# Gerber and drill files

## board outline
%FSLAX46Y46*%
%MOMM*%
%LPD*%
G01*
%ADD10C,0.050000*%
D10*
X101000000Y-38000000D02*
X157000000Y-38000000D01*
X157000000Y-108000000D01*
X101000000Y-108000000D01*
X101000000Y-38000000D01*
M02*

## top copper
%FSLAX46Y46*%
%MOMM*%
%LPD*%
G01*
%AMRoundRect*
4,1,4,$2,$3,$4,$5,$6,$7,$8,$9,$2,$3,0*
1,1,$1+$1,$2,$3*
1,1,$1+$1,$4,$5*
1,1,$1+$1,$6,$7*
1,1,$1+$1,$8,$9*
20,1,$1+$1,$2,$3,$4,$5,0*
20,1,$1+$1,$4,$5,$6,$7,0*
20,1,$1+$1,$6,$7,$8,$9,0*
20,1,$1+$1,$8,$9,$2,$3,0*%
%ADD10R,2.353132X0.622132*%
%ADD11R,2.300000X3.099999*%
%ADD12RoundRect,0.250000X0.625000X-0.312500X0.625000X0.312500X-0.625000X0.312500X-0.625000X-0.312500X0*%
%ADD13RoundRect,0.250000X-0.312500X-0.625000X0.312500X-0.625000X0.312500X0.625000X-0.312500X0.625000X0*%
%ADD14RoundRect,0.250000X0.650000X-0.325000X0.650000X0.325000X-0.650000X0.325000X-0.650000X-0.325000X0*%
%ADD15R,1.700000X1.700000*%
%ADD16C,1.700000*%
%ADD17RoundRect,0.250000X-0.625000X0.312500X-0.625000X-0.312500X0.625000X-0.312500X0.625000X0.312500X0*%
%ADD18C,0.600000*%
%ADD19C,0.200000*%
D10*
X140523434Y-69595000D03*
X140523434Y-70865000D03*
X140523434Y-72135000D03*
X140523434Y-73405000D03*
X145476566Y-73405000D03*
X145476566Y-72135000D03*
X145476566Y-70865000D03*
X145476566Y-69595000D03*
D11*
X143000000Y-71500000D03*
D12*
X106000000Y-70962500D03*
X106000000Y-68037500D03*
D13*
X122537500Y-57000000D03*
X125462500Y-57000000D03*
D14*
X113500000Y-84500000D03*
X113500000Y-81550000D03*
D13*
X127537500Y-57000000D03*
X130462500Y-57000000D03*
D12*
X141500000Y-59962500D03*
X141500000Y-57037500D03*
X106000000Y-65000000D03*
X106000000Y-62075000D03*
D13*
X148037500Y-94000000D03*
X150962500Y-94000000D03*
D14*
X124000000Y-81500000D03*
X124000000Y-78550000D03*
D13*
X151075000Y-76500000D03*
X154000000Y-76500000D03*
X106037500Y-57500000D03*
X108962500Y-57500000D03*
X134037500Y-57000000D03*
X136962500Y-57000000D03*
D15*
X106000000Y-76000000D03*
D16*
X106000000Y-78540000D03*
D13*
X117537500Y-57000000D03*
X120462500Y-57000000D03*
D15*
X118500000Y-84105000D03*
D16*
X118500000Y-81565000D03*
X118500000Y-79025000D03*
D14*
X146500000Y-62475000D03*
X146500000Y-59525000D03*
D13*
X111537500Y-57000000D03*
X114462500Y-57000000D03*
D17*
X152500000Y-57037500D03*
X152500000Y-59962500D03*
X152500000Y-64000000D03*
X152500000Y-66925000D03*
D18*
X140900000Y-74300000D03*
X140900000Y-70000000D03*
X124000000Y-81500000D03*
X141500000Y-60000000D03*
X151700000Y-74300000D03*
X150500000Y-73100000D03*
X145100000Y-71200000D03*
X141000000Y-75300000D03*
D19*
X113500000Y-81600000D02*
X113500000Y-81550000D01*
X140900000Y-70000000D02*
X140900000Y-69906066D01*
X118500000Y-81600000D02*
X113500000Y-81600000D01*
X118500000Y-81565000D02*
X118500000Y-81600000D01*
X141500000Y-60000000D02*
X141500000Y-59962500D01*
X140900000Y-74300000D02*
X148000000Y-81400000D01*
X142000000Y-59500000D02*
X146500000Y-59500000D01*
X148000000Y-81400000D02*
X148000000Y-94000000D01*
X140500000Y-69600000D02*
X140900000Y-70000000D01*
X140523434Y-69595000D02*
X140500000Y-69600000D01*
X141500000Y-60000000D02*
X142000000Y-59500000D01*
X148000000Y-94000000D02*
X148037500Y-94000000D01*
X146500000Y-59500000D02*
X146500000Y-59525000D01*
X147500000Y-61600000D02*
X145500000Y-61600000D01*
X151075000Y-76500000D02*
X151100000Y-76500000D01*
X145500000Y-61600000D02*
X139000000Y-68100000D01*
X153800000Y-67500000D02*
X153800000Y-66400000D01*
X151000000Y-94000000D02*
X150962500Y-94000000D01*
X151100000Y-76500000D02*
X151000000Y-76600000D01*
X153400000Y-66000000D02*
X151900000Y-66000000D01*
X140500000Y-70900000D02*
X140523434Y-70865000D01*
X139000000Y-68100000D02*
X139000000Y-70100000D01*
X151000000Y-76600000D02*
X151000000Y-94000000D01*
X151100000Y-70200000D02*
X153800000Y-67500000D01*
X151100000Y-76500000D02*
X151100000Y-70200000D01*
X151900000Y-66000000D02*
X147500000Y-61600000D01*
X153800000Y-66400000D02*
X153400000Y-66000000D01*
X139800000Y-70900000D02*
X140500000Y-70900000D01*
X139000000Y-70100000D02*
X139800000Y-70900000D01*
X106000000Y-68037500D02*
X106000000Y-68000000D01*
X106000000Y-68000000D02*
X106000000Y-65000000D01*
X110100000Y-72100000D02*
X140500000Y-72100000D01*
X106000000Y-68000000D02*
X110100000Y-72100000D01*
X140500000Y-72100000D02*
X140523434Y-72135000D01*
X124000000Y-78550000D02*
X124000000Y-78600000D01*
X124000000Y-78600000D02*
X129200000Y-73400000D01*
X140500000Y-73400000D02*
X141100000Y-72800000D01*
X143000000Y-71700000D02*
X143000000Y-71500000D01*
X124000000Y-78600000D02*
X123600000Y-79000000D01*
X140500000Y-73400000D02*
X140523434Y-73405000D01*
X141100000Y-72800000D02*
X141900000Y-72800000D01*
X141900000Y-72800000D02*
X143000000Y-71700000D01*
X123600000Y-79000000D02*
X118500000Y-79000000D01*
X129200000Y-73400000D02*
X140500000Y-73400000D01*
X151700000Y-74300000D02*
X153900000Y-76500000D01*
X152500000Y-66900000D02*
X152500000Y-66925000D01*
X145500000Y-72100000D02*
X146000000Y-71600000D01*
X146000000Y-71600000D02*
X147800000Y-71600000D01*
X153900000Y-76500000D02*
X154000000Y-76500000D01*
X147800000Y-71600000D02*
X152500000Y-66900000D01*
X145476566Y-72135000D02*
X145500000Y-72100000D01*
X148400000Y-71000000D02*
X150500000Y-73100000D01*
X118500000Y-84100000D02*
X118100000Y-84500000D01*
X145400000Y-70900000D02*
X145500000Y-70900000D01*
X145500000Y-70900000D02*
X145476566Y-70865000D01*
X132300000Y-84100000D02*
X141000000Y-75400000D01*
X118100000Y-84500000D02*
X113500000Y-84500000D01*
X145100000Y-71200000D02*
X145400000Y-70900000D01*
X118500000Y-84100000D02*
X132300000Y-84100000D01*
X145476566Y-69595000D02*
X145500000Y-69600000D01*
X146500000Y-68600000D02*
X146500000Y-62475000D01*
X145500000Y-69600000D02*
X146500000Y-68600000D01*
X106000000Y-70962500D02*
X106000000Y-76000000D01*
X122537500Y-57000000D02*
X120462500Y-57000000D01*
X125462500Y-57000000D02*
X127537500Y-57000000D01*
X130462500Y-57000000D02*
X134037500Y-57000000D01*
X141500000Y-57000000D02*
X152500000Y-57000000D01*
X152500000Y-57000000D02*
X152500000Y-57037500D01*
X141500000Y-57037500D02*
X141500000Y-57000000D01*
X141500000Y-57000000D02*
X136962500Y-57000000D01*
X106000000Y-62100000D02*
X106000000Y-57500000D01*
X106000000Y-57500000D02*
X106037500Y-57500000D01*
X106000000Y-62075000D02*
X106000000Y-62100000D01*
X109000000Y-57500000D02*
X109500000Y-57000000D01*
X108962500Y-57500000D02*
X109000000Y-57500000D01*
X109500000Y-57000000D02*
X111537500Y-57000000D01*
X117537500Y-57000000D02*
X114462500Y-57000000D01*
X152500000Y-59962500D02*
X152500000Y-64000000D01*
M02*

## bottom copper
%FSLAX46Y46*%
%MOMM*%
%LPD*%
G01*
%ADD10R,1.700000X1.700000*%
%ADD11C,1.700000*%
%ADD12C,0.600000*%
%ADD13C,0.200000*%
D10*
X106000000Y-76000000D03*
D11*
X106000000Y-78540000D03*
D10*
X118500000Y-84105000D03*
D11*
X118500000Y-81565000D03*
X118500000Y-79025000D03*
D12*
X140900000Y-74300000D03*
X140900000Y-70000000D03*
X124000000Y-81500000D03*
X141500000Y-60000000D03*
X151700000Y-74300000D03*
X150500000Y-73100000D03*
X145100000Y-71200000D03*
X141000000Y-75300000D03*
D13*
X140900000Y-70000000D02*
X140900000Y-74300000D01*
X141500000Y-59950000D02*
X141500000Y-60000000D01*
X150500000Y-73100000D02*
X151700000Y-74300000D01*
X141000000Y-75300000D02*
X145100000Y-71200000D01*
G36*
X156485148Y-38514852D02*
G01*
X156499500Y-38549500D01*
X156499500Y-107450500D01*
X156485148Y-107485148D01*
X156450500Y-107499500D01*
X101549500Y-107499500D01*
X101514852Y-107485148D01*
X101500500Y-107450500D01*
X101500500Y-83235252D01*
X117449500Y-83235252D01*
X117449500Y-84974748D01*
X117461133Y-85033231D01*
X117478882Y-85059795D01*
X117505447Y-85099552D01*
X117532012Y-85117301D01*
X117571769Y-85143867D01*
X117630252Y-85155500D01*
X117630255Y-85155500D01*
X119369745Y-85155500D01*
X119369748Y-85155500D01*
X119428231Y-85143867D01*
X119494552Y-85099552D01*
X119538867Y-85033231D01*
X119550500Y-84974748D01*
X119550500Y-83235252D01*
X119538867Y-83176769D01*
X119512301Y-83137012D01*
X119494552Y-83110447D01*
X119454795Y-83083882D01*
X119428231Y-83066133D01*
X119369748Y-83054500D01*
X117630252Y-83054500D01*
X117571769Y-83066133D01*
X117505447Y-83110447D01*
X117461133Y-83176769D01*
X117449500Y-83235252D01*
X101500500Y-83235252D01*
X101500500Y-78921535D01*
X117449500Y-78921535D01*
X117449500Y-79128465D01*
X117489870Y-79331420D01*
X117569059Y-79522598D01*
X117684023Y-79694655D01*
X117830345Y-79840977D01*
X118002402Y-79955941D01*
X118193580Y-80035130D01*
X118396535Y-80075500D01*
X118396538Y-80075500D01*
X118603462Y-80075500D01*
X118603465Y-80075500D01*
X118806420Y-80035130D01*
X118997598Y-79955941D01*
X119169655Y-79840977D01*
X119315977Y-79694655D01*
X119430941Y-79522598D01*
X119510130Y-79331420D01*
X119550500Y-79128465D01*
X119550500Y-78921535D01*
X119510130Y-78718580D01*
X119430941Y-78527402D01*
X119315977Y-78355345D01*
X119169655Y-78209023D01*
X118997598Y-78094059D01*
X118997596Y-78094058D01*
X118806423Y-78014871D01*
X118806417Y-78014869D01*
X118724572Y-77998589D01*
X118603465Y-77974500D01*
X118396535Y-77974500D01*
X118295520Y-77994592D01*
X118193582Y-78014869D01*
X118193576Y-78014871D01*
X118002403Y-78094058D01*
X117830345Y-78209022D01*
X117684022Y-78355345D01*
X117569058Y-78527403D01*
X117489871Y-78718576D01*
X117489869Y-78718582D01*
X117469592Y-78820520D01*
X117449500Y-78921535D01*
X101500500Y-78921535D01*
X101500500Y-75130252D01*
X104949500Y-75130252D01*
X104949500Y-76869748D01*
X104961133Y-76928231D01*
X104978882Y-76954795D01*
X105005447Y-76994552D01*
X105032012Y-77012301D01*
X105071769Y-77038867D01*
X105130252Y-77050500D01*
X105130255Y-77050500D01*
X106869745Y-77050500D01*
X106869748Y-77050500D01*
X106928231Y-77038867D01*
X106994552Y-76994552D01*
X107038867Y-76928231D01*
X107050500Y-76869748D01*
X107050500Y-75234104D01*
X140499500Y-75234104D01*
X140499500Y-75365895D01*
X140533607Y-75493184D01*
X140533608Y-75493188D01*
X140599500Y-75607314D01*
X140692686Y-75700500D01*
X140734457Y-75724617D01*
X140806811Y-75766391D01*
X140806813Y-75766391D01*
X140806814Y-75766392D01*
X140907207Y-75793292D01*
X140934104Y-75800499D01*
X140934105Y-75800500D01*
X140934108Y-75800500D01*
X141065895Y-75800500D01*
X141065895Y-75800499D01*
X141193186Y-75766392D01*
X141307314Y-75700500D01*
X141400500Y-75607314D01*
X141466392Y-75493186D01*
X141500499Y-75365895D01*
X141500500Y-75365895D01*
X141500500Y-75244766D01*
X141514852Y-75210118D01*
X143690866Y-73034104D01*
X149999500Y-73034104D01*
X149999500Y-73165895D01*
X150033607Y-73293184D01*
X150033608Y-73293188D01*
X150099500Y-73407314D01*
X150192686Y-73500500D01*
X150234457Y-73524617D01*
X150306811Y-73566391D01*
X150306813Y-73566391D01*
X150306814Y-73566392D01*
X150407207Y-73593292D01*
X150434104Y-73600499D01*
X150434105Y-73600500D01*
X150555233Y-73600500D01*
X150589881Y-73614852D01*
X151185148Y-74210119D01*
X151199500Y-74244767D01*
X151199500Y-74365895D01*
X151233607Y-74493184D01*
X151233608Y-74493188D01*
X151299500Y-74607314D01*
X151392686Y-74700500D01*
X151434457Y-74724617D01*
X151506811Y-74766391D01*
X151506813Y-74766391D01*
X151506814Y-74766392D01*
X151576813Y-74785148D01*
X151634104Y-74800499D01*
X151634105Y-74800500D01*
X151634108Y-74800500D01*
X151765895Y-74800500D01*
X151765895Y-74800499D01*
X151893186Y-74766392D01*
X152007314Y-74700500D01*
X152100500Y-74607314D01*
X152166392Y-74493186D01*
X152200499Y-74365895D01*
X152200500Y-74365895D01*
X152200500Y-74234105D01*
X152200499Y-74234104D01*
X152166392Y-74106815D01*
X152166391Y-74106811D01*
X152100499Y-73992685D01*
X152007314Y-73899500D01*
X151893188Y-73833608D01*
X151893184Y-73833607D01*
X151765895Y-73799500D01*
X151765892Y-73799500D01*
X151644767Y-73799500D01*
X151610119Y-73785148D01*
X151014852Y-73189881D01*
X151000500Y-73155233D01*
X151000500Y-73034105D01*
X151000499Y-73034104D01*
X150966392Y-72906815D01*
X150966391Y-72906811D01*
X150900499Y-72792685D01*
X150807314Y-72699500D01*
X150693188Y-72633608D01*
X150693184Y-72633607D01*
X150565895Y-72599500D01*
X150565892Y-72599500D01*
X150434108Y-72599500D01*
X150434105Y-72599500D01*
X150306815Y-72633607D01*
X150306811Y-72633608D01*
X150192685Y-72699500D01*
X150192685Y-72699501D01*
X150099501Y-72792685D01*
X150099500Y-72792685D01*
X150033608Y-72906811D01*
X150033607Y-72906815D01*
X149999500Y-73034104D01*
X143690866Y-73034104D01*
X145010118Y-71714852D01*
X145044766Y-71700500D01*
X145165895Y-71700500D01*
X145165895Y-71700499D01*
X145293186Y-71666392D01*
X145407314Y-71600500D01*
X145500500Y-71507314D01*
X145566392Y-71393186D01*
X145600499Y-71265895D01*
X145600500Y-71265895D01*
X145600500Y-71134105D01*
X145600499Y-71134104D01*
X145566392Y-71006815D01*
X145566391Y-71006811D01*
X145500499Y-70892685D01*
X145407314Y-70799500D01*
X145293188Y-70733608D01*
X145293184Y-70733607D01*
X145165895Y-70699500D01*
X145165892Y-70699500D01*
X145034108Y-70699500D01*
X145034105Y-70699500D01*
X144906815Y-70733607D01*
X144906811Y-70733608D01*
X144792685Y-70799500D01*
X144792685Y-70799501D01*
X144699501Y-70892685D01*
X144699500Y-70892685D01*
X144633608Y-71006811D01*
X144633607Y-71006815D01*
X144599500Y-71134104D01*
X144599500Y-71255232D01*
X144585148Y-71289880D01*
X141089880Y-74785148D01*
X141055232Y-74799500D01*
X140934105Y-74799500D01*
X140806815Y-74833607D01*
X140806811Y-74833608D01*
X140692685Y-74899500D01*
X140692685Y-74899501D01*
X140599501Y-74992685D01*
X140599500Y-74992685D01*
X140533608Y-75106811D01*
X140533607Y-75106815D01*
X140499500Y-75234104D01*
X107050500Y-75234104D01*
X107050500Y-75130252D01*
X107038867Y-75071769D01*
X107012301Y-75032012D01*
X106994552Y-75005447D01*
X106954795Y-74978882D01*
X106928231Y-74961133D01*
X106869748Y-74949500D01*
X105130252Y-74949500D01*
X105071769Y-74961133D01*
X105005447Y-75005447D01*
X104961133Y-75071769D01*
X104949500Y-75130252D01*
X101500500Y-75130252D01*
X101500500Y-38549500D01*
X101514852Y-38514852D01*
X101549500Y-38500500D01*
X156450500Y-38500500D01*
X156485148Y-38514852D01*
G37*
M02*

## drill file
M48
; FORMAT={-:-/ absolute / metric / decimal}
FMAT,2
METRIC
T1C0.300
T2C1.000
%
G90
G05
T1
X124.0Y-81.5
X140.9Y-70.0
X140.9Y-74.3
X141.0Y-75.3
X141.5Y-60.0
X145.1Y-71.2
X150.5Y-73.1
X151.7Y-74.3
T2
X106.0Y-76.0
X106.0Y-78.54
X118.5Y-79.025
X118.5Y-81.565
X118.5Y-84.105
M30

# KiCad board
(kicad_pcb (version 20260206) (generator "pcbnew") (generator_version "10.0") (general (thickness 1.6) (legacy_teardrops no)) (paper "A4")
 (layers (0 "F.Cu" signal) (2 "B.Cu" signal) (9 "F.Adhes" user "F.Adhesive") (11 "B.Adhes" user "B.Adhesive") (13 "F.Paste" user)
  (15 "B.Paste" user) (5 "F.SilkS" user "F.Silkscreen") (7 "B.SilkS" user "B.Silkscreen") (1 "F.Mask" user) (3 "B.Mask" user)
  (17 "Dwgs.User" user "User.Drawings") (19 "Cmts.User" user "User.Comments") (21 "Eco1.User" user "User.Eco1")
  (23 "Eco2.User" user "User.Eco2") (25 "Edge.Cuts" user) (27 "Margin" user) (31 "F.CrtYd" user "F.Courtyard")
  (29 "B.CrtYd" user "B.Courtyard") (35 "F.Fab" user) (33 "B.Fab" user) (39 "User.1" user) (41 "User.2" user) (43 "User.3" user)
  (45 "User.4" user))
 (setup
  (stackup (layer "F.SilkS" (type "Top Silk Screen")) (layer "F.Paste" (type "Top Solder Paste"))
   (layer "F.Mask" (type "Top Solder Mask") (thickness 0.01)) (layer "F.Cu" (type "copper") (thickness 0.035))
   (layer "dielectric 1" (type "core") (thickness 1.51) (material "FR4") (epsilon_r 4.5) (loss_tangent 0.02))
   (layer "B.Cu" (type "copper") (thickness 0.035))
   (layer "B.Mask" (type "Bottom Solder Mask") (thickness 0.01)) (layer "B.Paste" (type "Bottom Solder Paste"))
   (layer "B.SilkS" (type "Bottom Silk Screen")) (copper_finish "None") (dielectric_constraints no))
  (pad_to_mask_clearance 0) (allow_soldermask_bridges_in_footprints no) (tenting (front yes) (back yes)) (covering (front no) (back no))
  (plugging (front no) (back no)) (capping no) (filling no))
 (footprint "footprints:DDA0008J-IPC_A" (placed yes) (layer "F.Cu") (at 143 71.5)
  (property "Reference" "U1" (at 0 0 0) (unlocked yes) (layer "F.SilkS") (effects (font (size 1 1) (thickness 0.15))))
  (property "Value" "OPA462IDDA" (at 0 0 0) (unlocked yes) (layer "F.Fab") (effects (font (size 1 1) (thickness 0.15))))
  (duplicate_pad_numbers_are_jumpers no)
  (pad "1" smd rect (at -2.476566 -1.905) (size 2.353132 0.622132) (layers "F.Cu" "F.Mask" "F.Paste") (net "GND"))
  (pad "2" smd rect (at -2.476566 -0.635) (size 2.353132 0.622132) (layers "F.Cu" "F.Mask" "F.Paste") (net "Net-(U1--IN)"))
  (pad "3" smd rect (at -2.476566 0.635) (size 2.353132 0.622132) (layers "F.Cu" "F.Mask" "F.Paste") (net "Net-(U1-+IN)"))
  (pad "4" smd rect (at -2.476566 1.905) (size 2.353132 0.622132) (layers "F.Cu" "F.Mask" "F.Paste") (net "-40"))
  (pad "5" smd rect (at 2.476566 1.905) (size 2.353132 0.622132) (layers "F.Cu" "F.Mask" "F.Paste")
   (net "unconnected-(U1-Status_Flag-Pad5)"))
  (pad "6" smd rect (at 2.476566 0.635) (size 2.353132 0.622132) (layers "F.Cu" "F.Mask" "F.Paste") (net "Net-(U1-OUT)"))
  (pad "7" smd rect (at 2.476566 -0.635) (size 2.353132 0.622132) (layers "F.Cu" "F.Mask" "F.Paste") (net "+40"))
  (pad "8" smd rect (at 2.476566 -1.905) (size 2.353132 0.622132) (layers "F.Cu" "F.Mask" "F.Paste") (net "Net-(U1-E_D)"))
  (pad "9" smd rect (at 0 0) (size 2.3 3.099999) (layers "F.Cu" "F.Mask") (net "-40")))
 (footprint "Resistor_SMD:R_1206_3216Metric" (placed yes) (layer "F.Cu") (at 106 69.5 90)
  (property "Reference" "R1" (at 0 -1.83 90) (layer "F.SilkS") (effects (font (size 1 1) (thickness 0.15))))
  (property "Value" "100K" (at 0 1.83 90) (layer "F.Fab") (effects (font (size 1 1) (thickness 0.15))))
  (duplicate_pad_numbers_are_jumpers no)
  (pad "1" smd roundrect (at -1.4625 0 90) (size 1.125 1.75) (layers "F.Cu" "F.Mask" "F.Paste") (roundrect_rratio 0.222222)
   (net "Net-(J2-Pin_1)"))
  (pad "2" smd roundrect (at 1.4625 0 90) (size 1.125 1.75) (layers "F.Cu" "F.Mask" "F.Paste") (roundrect_rratio 0.222222)
   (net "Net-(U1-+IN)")))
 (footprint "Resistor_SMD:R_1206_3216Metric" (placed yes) (layer "F.Cu") (at 124 57)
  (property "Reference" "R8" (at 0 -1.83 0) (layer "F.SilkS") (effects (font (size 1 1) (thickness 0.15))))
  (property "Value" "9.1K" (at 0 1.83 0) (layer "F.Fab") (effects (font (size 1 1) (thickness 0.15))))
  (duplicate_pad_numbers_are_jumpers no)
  (pad "1" smd roundrect (at -1.4625 0) (size 1.125 1.75) (layers "F.Cu" "F.Mask" "F.Paste") (roundrect_rratio 0.222222)
   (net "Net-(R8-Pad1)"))
  (pad "2" smd roundrect (at 1.4625 0) (size 1.125 1.75) (layers "F.Cu" "F.Mask" "F.Paste") (roundrect_rratio 0.222222)
   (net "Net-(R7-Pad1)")))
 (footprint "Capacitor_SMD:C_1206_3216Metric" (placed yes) (layer "F.Cu") (at 113.5 83.025 90)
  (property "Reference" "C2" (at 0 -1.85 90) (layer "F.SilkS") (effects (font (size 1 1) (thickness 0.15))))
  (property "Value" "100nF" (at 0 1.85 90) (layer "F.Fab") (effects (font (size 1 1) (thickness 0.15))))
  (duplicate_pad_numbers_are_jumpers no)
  (pad "1" smd roundrect (at -1.475 0 90) (size 1.15 1.8) (layers "F.Cu" "F.Mask" "F.Paste") (roundrect_rratio 0.217391) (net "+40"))
  (pad "2" smd roundrect (at 1.475 0 90) (size 1.15 1.8) (layers "F.Cu" "F.Mask" "F.Paste") (roundrect_rratio 0.217391) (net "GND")))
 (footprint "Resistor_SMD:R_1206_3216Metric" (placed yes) (layer "F.Cu") (at 129 57)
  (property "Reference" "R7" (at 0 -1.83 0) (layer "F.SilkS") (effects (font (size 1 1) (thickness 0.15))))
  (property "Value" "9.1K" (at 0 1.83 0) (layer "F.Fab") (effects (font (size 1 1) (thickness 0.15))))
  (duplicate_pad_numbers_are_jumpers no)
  (pad "1" smd roundrect (at -1.4625 0) (size 1.125 1.75) (layers "F.Cu" "F.Mask" "F.Paste") (roundrect_rratio 0.222222)
   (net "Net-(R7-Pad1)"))
  (pad "2" smd roundrect (at 1.4625 0) (size 1.125 1.75) (layers "F.Cu" "F.Mask" "F.Paste") (roundrect_rratio 0.222222)
   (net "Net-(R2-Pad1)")))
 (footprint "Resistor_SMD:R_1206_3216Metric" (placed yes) (layer "F.Cu") (at 141.5 58.5 90)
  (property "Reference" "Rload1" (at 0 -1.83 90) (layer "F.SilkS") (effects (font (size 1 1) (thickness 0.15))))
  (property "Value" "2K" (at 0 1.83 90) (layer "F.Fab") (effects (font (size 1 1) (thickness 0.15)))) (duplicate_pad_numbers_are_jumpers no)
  (pad "1" smd roundrect (at -1.4625 0 90) (size 1.125 1.75) (layers "F.Cu" "F.Mask" "F.Paste") (roundrect_rratio 0.222222) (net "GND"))
  (pad "2" smd roundrect (at 1.4625 0 90) (size 1.125 1.75) (layers "F.Cu" "F.Mask" "F.Paste") (roundrect_rratio 0.222222)
   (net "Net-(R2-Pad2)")))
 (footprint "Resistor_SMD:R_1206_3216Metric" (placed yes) (layer "F.Cu") (at 106 63.5375 90)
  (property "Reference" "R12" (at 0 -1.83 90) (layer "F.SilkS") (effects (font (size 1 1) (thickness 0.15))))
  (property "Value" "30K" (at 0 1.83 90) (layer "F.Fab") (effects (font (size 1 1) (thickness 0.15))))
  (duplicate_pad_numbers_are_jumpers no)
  (pad "1" smd roundrect (at -1.4625 0 90) (size 1.125 1.75) (layers "F.Cu" "F.Mask" "F.Paste") (roundrect_rratio 0.222222)
   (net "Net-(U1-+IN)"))
  (pad "2" smd roundrect (at 1.4625 0 90) (size 1.125 1.75) (layers "F.Cu" "F.Mask" "F.Paste") (roundrect_rratio 0.222222)
   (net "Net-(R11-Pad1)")))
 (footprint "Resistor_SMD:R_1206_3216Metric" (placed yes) (layer "F.Cu") (at 149.5 94)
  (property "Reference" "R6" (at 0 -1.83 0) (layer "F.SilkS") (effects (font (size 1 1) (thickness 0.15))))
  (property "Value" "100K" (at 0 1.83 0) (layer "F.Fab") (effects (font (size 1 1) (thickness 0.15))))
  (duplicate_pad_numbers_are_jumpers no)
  (pad "1" smd roundrect (at -1.4625 0) (size 1.125 1.75) (layers "F.Cu" "F.Mask" "F.Paste") (roundrect_rratio 0.222222) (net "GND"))
  (pad "2" smd roundrect (at 1.4625 0) (size 1.125 1.75) (layers "F.Cu" "F.Mask" "F.Paste") (roundrect_rratio 0.222222) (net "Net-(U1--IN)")))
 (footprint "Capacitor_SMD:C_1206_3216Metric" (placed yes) (layer "F.Cu") (at 124 80.025 90)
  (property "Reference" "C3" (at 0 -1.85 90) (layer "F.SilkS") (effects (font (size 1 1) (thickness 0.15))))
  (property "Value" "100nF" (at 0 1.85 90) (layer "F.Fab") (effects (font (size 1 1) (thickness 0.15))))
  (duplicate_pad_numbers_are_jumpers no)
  (pad "1" smd roundrect (at -1.475 0 90) (size 1.15 1.8) (layers "F.Cu" "F.Mask" "F.Paste") (roundrect_rratio 0.217391) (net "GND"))
  (pad "2" smd roundrect (at 1.475 0 90) (size 1.15 1.8) (layers "F.Cu" "F.Mask" "F.Paste") (roundrect_rratio 0.217391) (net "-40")))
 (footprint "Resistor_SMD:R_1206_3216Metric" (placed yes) (layer "F.Cu") (at 152.5375 76.5)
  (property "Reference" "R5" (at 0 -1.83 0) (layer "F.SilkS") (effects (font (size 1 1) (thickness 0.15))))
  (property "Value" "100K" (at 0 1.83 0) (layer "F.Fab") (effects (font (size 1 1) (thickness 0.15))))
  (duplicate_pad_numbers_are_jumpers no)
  (pad "1" smd roundrect (at -1.4625 0) (size 1.125 1.75) (layers "F.Cu" "F.Mask" "F.Paste") (roundrect_rratio 0.222222)
   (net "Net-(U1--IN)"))
  (pad "2" smd roundrect (at 1.4625 0) (size 1.125 1.75) (layers "F.Cu" "F.Mask" "F.Paste") (roundrect_rratio 0.222222) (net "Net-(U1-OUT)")))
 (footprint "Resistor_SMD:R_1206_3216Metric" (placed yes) (layer "F.Cu") (at 107.5 57.5)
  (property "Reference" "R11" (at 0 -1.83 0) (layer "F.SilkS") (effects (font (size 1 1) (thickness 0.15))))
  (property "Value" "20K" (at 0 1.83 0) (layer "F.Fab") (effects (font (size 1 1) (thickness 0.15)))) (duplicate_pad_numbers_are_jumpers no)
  (pad "1" smd roundrect (at -1.4625 0) (size 1.125 1.75) (layers "F.Cu" "F.Mask" "F.Paste") (roundrect_rratio 0.222222)
   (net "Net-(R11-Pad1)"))
  (pad "2" smd roundrect (at 1.4625 0) (size 1.125 1.75) (layers "F.Cu" "F.Mask" "F.Paste") (roundrect_rratio 0.222222)
   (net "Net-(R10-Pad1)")))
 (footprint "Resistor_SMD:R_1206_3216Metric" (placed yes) (layer "F.Cu") (at 135.5 57)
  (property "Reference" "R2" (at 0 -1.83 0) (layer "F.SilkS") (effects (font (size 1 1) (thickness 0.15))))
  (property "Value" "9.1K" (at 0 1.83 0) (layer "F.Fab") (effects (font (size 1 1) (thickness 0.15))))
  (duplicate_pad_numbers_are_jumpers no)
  (pad "1" smd roundrect (at -1.4625 0) (size 1.125 1.75) (layers "F.Cu" "F.Mask" "F.Paste") (roundrect_rratio 0.222222)
   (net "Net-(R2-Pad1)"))
  (pad "2" smd roundrect (at 1.4625 0) (size 1.125 1.75) (layers "F.Cu" "F.Mask" "F.Paste") (roundrect_rratio 0.222222)
   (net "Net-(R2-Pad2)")))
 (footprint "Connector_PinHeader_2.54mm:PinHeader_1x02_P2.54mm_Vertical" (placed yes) (layer "F.Cu") (at 106 76)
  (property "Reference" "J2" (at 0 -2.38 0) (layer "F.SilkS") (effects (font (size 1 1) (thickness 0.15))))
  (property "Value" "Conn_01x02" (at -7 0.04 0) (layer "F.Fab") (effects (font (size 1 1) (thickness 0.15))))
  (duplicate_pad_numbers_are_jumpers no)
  (pad "1" thru_hole rect (at 0 0) (size 1.7 1.7) (drill 1) (layers "*.Cu" "*.Mask") (remove_unused_layers no) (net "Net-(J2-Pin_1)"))
  (pad "2" thru_hole circle (at 0 2.54) (size 1.7 1.7) (drill 1) (layers "*.Cu" "*.Mask") (remove_unused_layers no) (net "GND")))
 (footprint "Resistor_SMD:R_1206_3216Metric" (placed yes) (layer "F.Cu") (at 119 57)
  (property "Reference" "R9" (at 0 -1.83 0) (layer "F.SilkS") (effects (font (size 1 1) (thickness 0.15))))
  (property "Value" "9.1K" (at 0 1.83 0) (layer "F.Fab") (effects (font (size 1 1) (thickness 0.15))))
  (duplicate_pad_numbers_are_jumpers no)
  (pad "1" smd roundrect (at -1.4625 0) (size 1.125 1.75) (layers "F.Cu" "F.Mask" "F.Paste") (roundrect_rratio 0.222222)
   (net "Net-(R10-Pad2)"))
  (pad "2" smd roundrect (at 1.4625 0) (size 1.125 1.75) (layers "F.Cu" "F.Mask" "F.Paste") (roundrect_rratio 0.222222)
   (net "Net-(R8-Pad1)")))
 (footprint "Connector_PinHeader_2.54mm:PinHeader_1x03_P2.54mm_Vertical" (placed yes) (layer "F.Cu") (at 118.5 84.105 180)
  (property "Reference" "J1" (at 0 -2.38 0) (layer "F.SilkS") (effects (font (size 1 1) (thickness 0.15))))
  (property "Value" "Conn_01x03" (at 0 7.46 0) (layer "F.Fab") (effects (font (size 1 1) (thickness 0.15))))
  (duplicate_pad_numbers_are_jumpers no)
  (pad "1" thru_hole rect (at 0 0 180) (size 1.7 1.7) (drill 1) (layers "*.Cu" "*.Mask") (remove_unused_layers no) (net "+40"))
  (pad "2" thru_hole circle (at 0 2.54 180) (size 1.7 1.7) (drill 1) (layers "*.Cu" "*.Mask") (remove_unused_layers no) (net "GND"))
  (pad "3" thru_hole circle (at 0 5.08 180) (size 1.7 1.7) (drill 1) (layers "*.Cu" "*.Mask") (remove_unused_layers no) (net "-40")))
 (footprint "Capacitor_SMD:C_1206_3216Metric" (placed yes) (layer "F.Cu") (at 146.5 61 90)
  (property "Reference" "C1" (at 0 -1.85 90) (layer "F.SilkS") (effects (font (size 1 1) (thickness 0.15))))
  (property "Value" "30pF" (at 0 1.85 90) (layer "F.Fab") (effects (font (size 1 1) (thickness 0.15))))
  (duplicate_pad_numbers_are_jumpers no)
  (pad "1" smd roundrect (at -1.475 0 90) (size 1.15 1.8) (layers "F.Cu" "F.Mask" "F.Paste") (roundrect_rratio 0.217391)
   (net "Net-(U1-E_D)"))
  (pad "2" smd roundrect (at 1.475 0 90) (size 1.15 1.8) (layers "F.Cu" "F.Mask" "F.Paste") (roundrect_rratio 0.217391) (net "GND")))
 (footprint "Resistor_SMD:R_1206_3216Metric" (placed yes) (layer "F.Cu") (at 113 57)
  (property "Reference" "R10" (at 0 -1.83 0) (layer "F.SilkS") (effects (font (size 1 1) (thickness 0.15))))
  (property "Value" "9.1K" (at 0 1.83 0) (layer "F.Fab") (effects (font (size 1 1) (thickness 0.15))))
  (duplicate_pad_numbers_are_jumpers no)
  (pad "1" smd roundrect (at -1.4625 0) (size 1.125 1.75) (layers "F.Cu" "F.Mask" "F.Paste") (roundrect_rratio 0.222222)
   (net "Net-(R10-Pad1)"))
  (pad "2" smd roundrect (at 1.4625 0) (size 1.125 1.75) (layers "F.Cu" "F.Mask" "F.Paste") (roundrect_rratio 0.222222)
   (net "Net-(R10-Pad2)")))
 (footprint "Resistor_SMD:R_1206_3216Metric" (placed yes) (layer "F.Cu") (at 152.5 58.5 -90)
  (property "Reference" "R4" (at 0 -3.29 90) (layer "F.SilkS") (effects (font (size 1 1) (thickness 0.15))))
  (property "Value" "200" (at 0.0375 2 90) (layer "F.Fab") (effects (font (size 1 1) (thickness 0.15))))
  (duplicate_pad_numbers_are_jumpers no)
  (pad "1" smd roundrect (at -1.4625 0 270) (size 1.125 1.75) (layers "F.Cu" "F.Mask" "F.Paste") (roundrect_rratio 0.222222)
   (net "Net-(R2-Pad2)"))
  (pad "2" smd roundrect (at 1.4625 0 270) (size 1.125 1.75) (layers "F.Cu" "F.Mask" "F.Paste") (roundrect_rratio 0.222222)
   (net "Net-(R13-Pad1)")))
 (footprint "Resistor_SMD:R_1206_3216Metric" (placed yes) (layer "F.Cu") (at 152.5 65.4625 -90)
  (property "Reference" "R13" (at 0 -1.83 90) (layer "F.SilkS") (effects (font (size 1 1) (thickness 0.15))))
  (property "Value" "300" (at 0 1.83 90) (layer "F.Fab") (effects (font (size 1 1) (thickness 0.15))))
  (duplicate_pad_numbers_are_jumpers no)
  (pad "1" smd roundrect (at -1.4625 0 270) (size 1.125 1.75) (layers "F.Cu" "F.Mask" "F.Paste") (roundrect_rratio 0.222222)
   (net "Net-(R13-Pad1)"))
  (pad "2" smd roundrect (at 1.4625 0 270) (size 1.125 1.75) (layers "F.Cu" "F.Mask" "F.Paste") (roundrect_rratio 0.222222)
   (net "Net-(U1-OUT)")))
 (gr_rect (start 101 38) (end 157 108) (stroke (width 0.05) (type default)) (fill no) (layer "Edge.Cuts"))
 (segment (start 113.5 81.6) (end 113.5 81.55) (width 0.2) (layer "F.Cu") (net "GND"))
 (segment (start 140.9 70) (end 140.9 69.906066) (width 0.2) (layer "F.Cu") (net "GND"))
 (segment (start 118.5 81.6) (end 113.5 81.6) (width 0.2) (layer "F.Cu") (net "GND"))
 (segment (start 118.5 81.565) (end 118.5 81.6) (width 0.2) (layer "F.Cu") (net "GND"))
 (segment (start 141.5 60) (end 141.5 59.9625) (width 0.2) (layer "F.Cu") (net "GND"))
 (segment (start 140.9 74.3) (end 148 81.4) (width 0.2) (layer "F.Cu") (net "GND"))
 (segment (start 142 59.5) (end 146.5 59.5) (width 0.2) (layer "F.Cu") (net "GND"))
 (segment (start 148 81.4) (end 148 94) (width 0.2) (layer "F.Cu") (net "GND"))
 (segment (start 140.5 69.6) (end 140.9 70) (width 0.2) (layer "F.Cu") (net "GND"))
 (segment (start 140.523434 69.595) (end 140.5 69.6) (width 0.2) (layer "F.Cu") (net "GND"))
 (segment (start 141.5 60) (end 142 59.5) (width 0.2) (layer "F.Cu") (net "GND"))
 (segment (start 148 94) (end 148.0375 94) (width 0.2) (layer "F.Cu") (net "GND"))
 (segment (start 146.5 59.5) (end 146.5 59.525) (width 0.2) (layer "F.Cu") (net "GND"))
 (via (at 140.9 74.3) (size 0.6) (drill 0.3) (layers "F.Cu" "B.Cu") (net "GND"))
 (via (at 140.9 70) (size 0.6) (drill 0.3) (layers "F.Cu" "B.Cu") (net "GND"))
 (via (at 124 81.5) (size 0.6) (drill 0.3) (layers "F.Cu" "B.Cu") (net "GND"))
 (via (at 141.5 60) (size 0.6) (drill 0.3) (layers "F.Cu" "B.Cu") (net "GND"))
 (segment (start 140.9 70) (end 140.9 74.3) (width 0.2) (layer "B.Cu") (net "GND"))
 (segment (start 141.5 59.95) (end 141.5 60) (width 0.2) (layer "B.Cu") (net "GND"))
 (segment (start 147.5 61.6) (end 145.5 61.6) (width 0.2) (layer "F.Cu") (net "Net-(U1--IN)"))
 (segment (start 151.075 76.5) (end 151.1 76.5) (width 0.2) (layer "F.Cu") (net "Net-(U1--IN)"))
 (segment (start 145.5 61.6) (end 139 68.1) (width 0.2) (layer "F.Cu") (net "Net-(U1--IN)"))
 (segment (start 153.8 67.5) (end 153.8 66.4) (width 0.2) (layer "F.Cu") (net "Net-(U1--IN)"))
 (segment (start 151 94) (end 150.9625 94) (width 0.2) (layer "F.Cu") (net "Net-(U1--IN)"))
 (segment (start 151.1 76.5) (end 151 76.6) (width 0.2) (layer "F.Cu") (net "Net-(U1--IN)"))
 (segment (start 153.4 66) (end 151.9 66) (width 0.2) (layer "F.Cu") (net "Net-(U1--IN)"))
 (segment (start 140.5 70.9) (end 140.523434 70.865) (width 0.2) (layer "F.Cu") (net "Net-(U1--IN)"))
 (segment (start 139 68.1) (end 139 70.1) (width 0.2) (layer "F.Cu") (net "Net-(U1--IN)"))
 (segment (start 151 76.6) (end 151 94) (width 0.2) (layer "F.Cu") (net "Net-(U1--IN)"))
 (segment (start 151.1 70.2) (end 153.8 67.5) (width 0.2) (layer "F.Cu") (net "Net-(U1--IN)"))
 (segment (start 151.1 76.5) (end 151.1 70.2) (width 0.2) (layer "F.Cu") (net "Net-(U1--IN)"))
 (segment (start 151.9 66) (end 147.5 61.6) (width 0.2) (layer "F.Cu") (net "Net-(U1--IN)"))
 (segment (start 153.8 66.4) (end 153.4 66) (width 0.2) (layer "F.Cu") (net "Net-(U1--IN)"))
 (segment (start 139.8 70.9) (end 140.5 70.9) (width 0.2) (layer "F.Cu") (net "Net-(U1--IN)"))
 (segment (start 139 70.1) (end 139.8 70.9) (width 0.2) (layer "F.Cu") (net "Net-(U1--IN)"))
 (segment (start 106 68.0375) (end 106 68) (width 0.2) (layer "F.Cu") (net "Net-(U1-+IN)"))
 (segment (start 106 68) (end 106 65) (width 0.2) (layer "F.Cu") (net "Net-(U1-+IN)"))
 (segment (start 110.1 72.1) (end 140.5 72.1) (width 0.2) (layer "F.Cu") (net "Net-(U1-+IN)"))
 (segment (start 106 68) (end 110.1 72.1) (width 0.2) (layer "F.Cu") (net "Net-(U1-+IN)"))
 (segment (start 140.5 72.1) (end 140.523434 72.135) (width 0.2) (layer "F.Cu") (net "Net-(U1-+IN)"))
 (segment (start 124 78.55) (end 124 78.6) (width 0.2) (layer "F.Cu") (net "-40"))
 (segment (start 124 78.6) (end 129.2 73.4) (width 0.2) (layer "F.Cu") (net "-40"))
 (segment (start 140.5 73.4) (end 141.1 72.8) (width 0.2) (layer "F.Cu") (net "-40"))
 (segment (start 143 71.7) (end 143 71.5) (width 0.2) (layer "F.Cu") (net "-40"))
 (segment (start 124 78.6) (end 123.6 79) (width 0.2) (layer "F.Cu") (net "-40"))
 (segment (start 140.5 73.4) (end 140.523434 73.405) (width 0.2) (layer "F.Cu") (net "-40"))
 (segment (start 141.1 72.8) (end 141.9 72.8) (width 0.2) (layer "F.Cu") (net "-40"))
 (segment (start 141.9 72.8) (end 143 71.7) (width 0.2) (layer "F.Cu") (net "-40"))
 (segment (start 123.6 79) (end 118.5 79) (width 0.2) (layer "F.Cu") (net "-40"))
 (segment (start 129.2 73.4) (end 140.5 73.4) (width 0.2) (layer "F.Cu") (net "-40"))
 (segment (start 151.7 74.3) (end 153.9 76.5) (width 0.2) (layer "F.Cu") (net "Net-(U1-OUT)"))
 (segment (start 152.5 66.9) (end 152.5 66.925) (width 0.2) (layer "F.Cu") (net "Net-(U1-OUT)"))
 (segment (start 145.5 72.1) (end 146 71.6) (width 0.2) (layer "F.Cu") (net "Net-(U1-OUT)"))
 (segment (start 146 71.6) (end 147.8 71.6) (width 0.2) (layer "F.Cu") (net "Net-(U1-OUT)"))
 (segment (start 153.9 76.5) (end 154 76.5) (width 0.2) (layer "F.Cu") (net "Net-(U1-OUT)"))
 (segment (start 147.8 71.6) (end 152.5 66.9) (width 0.2) (layer "F.Cu") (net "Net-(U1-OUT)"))
 (segment (start 145.476566 72.135) (end 145.5 72.1) (width 0.2) (layer "F.Cu") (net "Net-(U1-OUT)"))
 (segment (start 148.4 71) (end 150.5 73.1) (width 0.2) (layer "F.Cu") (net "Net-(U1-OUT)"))
 (via (at 151.7 74.3) (size 0.6) (drill 0.3) (layers "F.Cu" "B.Cu") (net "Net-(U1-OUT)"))
 (via (at 150.5 73.1) (size 0.6) (drill 0.3) (layers "F.Cu" "B.Cu") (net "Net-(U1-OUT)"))
 (segment (start 150.5 73.1) (end 151.7 74.3) (width 0.2) (layer "B.Cu") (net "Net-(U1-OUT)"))
 (segment (start 118.5 84.1) (end 118.1 84.5) (width 0.2) (layer "F.Cu") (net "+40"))
 (segment (start 145.4 70.9) (end 145.5 70.9) (width 0.2) (layer "F.Cu") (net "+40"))
 (segment (start 145.5 70.9) (end 145.476566 70.865) (width 0.2) (layer "F.Cu") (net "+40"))
 (segment (start 132.3 84.1) (end 141 75.4) (width 0.2) (layer "F.Cu") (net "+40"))
 (segment (start 118.1 84.5) (end 113.5 84.5) (width 0.2) (layer "F.Cu") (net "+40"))
 (segment (start 145.1 71.2) (end 145.4 70.9) (width 0.2) (layer "F.Cu") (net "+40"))
 (segment (start 118.5 84.1) (end 132.3 84.1) (width 0.2) (layer "F.Cu") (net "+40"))
 (via (at 145.1 71.2) (size 0.6) (drill 0.3) (layers "F.Cu" "B.Cu") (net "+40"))
 (via (at 141 75.3) (size 0.6) (drill 0.3) (layers "F.Cu" "B.Cu") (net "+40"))
 (segment (start 141 75.3) (end 145.1 71.2) (width 0.2) (layer "B.Cu") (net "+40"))
 (segment (start 145.476566 69.595) (end 145.5 69.6) (width 0.2) (layer "F.Cu") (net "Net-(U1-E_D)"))
 (segment (start 146.5 68.6) (end 146.5 62.475) (width 0.2) (layer "F.Cu") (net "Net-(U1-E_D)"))
 (segment (start 145.5 69.6) (end 146.5 68.6) (width 0.2) (layer "F.Cu") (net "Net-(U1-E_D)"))
 (segment (start 106 70.9625) (end 106 76) (width 0.2) (layer "F.Cu") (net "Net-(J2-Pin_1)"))
 (segment (start 122.5375 57) (end 120.4625 57) (width 0.2) (layer "F.Cu") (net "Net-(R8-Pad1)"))
 (segment (start 125.4625 57) (end 127.5375 57) (width 0.2) (layer "F.Cu") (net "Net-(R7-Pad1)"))
 (segment (start 130.4625 57) (end 134.0375 57) (width 0.2) (layer "F.Cu") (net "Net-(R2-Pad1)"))
 (segment (start 141.5 57) (end 152.5 57) (width 0.2) (layer "F.Cu") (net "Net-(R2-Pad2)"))
 (segment (start 152.5 57) (end 152.5 57.0375) (width 0.2) (layer "F.Cu") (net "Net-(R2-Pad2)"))
 (segment (start 141.5 57.0375) (end 141.5 57) (width 0.2) (layer "F.Cu") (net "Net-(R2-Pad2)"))
 (segment (start 141.5 57) (end 136.9625 57) (width 0.2) (layer "F.Cu") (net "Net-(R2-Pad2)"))
 (segment (start 106 62.1) (end 106 57.5) (width 0.2) (layer "F.Cu") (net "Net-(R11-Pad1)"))
 (segment (start 106 57.5) (end 106.0375 57.5) (width 0.2) (layer "F.Cu") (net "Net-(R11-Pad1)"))
 (segment (start 106 62.075) (end 106 62.1) (width 0.2) (layer "F.Cu") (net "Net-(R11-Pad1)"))
 (segment (start 109 57.5) (end 109.5 57) (width 0.2) (layer "F.Cu") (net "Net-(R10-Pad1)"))
 (segment (start 108.9625 57.5) (end 109 57.5) (width 0.2) (layer "F.Cu") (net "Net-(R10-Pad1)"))
 (segment (start 109.5 57) (end 111.5375 57) (width 0.2) (layer "F.Cu") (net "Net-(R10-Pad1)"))
 (segment (start 117.5375 57) (end 114.4625 57) (width 0.2) (layer "F.Cu") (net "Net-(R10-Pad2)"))
 (segment (start 152.5 59.9625) (end 152.5 64) (width 0.2) (layer "F.Cu") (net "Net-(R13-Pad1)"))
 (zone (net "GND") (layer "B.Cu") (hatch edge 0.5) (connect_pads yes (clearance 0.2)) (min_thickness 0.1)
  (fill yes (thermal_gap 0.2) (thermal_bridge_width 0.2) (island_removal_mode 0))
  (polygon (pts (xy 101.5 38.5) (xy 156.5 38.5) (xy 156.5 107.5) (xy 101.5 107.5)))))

